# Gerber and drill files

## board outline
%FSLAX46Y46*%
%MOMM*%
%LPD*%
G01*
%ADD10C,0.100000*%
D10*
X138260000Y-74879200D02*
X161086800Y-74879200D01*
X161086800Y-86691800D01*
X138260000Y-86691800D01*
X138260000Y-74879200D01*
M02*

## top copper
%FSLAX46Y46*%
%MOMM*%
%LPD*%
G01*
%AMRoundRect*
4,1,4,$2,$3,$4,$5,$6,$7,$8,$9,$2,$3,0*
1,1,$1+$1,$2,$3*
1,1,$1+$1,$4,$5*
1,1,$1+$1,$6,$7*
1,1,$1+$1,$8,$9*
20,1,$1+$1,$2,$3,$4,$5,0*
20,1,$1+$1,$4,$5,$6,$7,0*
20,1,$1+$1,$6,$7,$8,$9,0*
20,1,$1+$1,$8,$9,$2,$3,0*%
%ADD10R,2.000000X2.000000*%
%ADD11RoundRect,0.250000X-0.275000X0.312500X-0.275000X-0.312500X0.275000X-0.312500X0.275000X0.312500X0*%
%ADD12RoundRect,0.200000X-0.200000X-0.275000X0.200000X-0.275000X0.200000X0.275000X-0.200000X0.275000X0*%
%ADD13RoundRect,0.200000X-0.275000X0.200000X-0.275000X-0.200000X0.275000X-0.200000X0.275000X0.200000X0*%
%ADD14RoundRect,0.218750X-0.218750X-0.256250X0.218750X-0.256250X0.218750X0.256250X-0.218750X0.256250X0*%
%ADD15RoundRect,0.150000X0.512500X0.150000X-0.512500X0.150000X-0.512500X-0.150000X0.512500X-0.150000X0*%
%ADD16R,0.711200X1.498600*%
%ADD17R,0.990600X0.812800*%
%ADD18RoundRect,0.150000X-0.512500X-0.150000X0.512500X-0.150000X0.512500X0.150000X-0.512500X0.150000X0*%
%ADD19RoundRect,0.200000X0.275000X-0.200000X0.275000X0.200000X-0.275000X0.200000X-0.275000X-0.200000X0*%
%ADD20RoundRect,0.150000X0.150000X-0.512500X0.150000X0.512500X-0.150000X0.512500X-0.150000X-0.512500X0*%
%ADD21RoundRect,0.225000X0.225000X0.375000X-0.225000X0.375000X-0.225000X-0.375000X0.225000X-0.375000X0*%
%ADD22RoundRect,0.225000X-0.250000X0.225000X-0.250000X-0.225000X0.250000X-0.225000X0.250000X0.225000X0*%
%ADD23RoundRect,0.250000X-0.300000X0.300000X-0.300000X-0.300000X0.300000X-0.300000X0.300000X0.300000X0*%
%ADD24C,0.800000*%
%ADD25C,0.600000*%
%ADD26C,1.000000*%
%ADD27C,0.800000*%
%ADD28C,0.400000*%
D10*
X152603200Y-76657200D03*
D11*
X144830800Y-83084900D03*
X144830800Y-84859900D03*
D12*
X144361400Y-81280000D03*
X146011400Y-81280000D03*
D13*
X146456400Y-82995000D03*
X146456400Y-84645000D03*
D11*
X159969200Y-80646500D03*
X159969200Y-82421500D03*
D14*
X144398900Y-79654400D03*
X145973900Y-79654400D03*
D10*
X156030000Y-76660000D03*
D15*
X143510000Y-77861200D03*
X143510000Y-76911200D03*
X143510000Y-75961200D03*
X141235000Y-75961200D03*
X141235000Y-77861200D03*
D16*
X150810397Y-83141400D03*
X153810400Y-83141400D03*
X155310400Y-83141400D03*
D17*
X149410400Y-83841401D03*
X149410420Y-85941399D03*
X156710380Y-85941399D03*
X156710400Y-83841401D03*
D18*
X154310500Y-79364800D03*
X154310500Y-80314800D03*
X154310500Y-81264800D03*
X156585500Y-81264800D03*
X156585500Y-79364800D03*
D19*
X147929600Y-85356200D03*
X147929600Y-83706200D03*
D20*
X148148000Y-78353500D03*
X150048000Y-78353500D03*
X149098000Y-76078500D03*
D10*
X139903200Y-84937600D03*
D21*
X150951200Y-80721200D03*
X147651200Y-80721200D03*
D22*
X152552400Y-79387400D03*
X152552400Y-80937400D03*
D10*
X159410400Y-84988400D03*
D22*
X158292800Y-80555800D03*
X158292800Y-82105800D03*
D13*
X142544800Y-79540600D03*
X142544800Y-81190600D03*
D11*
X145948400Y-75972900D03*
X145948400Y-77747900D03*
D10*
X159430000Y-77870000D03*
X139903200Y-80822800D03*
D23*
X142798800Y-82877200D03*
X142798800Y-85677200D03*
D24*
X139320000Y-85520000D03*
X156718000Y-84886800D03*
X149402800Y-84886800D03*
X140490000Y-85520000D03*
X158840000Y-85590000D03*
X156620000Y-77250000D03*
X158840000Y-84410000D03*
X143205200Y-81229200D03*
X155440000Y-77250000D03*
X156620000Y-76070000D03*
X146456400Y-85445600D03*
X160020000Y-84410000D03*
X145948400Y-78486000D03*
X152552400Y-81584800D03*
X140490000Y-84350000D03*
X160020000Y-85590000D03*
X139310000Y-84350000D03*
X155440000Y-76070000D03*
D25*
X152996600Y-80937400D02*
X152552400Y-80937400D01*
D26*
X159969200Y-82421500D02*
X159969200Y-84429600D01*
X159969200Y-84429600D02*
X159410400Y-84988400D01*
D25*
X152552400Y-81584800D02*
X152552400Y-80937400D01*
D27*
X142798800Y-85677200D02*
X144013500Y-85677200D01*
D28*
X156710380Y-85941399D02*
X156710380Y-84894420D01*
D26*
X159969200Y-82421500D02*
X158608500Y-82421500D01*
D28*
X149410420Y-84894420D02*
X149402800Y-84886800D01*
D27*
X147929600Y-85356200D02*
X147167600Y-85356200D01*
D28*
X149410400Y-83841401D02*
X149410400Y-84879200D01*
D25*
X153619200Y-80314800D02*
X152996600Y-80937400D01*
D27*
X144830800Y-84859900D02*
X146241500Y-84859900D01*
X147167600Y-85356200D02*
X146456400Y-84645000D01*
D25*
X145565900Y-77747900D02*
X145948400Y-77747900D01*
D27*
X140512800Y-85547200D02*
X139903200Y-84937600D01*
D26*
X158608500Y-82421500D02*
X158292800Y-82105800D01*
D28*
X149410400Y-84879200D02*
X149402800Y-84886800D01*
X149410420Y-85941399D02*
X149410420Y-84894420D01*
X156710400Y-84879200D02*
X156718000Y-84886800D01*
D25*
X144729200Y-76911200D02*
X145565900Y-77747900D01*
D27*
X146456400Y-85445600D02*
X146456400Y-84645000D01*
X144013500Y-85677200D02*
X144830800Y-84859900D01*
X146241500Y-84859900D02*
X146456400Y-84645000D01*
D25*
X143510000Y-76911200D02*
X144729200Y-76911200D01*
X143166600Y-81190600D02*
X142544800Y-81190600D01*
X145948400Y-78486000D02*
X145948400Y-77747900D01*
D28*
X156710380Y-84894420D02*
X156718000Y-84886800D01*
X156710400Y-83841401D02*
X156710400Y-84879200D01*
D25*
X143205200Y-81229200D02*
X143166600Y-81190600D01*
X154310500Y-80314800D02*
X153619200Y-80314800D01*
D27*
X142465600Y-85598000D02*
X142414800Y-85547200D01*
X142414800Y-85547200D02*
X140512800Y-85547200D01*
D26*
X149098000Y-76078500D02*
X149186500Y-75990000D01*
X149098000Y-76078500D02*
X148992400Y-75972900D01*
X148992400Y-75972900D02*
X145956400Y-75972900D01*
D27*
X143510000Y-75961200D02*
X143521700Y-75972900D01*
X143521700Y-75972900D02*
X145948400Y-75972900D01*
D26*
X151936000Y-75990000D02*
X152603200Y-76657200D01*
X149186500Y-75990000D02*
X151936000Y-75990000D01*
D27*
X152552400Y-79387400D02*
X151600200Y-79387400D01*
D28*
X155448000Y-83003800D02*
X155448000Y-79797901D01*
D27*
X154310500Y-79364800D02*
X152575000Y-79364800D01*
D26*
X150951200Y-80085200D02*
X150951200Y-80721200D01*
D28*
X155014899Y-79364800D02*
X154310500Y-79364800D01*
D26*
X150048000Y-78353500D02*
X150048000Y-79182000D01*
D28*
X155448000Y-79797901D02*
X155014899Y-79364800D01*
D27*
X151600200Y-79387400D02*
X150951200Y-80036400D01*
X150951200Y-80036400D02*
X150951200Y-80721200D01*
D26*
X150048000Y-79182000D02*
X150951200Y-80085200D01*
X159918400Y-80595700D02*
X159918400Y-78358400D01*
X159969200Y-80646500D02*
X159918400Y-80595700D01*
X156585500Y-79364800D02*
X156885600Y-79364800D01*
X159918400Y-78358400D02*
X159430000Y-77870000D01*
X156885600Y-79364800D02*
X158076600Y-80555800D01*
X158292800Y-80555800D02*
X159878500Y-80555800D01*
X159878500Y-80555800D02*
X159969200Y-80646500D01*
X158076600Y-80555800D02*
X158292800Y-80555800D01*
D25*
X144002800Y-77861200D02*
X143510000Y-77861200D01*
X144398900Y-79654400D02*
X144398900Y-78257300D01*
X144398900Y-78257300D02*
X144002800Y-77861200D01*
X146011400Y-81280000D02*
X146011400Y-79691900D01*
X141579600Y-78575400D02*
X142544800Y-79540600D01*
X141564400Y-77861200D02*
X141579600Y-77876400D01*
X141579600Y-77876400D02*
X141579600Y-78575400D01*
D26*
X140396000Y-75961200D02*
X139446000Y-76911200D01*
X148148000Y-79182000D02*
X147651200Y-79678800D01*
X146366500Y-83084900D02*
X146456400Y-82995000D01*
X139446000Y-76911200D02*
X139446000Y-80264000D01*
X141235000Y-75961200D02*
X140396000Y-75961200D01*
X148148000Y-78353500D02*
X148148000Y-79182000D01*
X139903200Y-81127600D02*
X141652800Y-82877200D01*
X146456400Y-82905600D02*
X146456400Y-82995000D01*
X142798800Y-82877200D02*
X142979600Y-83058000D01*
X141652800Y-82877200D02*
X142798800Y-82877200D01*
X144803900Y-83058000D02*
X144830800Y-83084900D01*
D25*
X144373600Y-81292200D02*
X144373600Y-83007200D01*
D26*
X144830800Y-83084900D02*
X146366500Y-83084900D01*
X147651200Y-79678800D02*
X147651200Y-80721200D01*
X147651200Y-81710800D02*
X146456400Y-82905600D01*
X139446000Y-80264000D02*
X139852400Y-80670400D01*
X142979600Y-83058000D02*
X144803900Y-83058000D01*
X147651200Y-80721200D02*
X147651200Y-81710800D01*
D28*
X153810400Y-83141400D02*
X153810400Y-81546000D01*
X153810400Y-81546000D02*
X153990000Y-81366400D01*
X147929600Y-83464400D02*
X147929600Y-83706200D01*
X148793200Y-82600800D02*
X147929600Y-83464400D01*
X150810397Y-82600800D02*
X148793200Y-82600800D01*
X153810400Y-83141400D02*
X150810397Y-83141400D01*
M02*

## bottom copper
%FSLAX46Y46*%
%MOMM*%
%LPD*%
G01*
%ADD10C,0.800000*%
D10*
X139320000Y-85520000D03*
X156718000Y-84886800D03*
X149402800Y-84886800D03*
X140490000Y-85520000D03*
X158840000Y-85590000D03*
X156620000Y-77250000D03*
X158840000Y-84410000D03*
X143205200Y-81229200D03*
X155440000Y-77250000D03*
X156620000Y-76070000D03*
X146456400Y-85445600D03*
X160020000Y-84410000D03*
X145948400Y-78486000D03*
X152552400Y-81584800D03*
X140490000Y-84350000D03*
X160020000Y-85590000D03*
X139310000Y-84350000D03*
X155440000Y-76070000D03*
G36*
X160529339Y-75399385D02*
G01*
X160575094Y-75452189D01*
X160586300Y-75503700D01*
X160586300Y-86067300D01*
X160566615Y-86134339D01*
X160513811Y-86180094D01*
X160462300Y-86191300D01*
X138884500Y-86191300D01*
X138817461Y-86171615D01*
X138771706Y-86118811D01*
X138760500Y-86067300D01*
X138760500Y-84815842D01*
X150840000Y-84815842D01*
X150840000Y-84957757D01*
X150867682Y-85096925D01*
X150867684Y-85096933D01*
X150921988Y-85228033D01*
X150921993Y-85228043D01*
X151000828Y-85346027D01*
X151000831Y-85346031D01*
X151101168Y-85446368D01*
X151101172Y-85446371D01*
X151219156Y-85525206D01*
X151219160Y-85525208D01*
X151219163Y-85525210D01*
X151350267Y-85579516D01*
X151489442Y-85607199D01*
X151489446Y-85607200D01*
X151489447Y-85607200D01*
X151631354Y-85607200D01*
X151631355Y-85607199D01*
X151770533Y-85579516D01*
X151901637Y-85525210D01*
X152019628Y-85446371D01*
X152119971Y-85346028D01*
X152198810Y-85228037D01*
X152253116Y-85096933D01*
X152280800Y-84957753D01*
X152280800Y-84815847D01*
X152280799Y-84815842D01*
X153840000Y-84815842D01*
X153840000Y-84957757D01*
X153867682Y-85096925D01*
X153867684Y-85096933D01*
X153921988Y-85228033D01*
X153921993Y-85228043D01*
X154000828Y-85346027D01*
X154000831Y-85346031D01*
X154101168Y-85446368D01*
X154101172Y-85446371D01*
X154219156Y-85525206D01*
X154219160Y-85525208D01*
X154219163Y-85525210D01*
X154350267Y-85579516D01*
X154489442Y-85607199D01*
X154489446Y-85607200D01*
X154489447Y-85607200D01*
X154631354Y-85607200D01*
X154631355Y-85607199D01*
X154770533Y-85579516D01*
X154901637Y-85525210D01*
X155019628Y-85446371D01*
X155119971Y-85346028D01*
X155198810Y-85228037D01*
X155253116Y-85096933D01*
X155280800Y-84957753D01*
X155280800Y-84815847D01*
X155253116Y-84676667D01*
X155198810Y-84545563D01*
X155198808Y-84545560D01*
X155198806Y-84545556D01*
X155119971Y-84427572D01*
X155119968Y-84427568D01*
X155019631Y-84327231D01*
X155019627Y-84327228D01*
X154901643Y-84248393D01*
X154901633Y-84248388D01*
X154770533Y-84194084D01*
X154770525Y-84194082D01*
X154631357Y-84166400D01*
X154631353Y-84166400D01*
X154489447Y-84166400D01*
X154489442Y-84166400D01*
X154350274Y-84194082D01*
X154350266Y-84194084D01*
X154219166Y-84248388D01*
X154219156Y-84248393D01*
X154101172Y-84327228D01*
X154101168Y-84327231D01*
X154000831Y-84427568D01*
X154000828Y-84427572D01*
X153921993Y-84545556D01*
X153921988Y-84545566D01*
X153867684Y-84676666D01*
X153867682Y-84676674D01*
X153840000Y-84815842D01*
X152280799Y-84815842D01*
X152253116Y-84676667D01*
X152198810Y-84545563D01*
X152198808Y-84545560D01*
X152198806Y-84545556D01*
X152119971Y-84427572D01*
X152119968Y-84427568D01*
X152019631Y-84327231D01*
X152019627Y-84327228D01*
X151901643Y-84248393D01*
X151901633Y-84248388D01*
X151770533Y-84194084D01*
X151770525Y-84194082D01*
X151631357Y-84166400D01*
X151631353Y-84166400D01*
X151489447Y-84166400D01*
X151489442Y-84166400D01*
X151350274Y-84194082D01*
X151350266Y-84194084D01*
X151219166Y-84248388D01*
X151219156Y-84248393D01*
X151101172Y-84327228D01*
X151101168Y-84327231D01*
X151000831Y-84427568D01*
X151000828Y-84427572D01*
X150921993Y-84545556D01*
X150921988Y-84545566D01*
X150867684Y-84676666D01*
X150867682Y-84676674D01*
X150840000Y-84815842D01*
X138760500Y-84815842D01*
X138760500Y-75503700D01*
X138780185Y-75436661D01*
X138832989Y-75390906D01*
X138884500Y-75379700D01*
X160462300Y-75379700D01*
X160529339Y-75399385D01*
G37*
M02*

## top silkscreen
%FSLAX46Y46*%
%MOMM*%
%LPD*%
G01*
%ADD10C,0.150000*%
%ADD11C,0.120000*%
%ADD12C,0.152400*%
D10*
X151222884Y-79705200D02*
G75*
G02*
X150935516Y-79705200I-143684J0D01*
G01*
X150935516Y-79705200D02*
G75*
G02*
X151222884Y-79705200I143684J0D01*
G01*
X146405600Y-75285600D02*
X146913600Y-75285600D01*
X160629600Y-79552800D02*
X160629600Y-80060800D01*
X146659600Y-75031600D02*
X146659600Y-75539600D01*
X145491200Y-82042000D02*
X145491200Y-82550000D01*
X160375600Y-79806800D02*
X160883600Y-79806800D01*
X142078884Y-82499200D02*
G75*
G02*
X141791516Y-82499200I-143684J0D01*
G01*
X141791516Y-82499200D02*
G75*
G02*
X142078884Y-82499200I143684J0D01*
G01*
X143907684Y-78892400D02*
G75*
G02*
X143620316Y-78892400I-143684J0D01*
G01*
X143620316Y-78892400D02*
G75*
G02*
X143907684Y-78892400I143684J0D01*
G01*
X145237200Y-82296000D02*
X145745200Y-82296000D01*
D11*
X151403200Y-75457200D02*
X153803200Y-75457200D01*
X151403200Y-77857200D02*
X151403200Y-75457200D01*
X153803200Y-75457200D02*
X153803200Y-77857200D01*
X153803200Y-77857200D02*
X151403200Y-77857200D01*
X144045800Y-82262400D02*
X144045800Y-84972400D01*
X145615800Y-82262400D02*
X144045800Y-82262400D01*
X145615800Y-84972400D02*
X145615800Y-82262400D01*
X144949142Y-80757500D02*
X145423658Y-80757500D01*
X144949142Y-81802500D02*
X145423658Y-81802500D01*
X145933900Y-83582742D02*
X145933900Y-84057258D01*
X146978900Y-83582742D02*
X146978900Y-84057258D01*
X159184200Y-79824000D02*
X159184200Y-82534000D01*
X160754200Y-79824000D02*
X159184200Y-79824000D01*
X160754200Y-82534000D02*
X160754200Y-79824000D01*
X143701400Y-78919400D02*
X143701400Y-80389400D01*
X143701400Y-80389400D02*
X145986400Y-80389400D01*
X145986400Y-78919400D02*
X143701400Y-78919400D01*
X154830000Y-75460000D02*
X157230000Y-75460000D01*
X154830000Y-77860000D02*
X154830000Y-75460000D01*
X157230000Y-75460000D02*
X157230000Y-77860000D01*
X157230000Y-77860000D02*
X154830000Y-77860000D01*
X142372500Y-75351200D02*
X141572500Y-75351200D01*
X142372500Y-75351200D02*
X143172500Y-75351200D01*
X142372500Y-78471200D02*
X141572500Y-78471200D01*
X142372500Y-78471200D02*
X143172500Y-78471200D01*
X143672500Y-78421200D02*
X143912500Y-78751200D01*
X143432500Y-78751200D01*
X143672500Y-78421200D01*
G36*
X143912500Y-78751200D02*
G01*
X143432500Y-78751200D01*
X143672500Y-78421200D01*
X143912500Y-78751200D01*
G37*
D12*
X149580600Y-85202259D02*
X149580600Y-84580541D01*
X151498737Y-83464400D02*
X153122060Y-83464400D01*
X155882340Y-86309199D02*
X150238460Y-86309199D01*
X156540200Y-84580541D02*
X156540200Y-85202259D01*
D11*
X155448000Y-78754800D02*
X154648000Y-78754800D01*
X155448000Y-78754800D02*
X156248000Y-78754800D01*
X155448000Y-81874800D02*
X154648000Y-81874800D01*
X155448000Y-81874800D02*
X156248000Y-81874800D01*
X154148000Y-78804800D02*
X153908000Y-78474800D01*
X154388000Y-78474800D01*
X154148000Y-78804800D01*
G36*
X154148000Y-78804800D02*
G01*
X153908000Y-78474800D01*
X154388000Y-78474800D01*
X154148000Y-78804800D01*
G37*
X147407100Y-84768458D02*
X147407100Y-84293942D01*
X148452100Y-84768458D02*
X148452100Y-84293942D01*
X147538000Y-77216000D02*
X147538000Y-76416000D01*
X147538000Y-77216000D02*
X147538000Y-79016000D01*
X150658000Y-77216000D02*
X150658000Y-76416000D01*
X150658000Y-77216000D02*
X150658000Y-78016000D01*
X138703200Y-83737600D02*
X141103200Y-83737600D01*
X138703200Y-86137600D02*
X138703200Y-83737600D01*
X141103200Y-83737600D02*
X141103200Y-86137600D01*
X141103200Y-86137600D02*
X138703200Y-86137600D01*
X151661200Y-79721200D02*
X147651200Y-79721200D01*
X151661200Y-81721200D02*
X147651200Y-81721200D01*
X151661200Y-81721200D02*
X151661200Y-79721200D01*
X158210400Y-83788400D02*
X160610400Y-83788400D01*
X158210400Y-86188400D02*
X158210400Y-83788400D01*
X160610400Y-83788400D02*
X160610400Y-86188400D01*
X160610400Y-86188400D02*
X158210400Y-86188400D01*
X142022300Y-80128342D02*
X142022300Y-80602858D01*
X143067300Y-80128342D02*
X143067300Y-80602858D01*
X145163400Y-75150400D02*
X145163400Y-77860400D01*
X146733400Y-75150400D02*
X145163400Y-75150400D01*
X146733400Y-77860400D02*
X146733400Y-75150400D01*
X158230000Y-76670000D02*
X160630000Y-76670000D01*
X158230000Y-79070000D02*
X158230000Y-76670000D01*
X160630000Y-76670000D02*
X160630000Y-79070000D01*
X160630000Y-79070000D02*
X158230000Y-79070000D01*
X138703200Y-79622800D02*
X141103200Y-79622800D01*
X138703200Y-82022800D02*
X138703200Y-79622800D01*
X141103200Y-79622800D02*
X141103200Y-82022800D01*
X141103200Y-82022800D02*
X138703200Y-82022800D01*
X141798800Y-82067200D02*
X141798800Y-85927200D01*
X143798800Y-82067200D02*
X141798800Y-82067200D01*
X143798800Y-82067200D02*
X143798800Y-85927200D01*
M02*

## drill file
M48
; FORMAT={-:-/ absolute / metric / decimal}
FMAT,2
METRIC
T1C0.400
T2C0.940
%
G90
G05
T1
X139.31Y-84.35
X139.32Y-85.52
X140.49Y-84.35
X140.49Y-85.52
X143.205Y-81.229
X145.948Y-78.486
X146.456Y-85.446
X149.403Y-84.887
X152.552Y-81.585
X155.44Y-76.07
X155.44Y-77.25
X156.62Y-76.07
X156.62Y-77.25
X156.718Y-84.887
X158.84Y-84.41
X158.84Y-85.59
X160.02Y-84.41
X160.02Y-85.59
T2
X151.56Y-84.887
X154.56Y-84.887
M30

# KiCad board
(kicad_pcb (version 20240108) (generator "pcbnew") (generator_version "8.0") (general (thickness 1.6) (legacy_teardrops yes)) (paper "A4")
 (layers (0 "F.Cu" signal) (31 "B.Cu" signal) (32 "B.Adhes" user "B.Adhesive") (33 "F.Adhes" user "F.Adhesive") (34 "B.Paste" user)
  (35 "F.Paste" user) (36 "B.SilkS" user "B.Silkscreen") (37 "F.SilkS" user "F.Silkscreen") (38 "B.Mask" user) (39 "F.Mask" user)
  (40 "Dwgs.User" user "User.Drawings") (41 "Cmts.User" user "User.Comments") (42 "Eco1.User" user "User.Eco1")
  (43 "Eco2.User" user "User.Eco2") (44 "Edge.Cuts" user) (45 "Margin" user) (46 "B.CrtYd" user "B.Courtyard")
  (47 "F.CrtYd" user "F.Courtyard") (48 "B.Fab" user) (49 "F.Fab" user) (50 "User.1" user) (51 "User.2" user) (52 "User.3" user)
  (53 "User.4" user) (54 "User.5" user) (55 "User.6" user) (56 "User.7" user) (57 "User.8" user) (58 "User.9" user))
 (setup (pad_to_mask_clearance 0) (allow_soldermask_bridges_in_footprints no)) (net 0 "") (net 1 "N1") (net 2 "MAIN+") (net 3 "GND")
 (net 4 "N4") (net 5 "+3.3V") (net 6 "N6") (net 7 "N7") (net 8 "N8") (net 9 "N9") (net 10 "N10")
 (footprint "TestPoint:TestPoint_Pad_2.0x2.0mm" (layer "F.Cu") (at 152.6032 76.6572)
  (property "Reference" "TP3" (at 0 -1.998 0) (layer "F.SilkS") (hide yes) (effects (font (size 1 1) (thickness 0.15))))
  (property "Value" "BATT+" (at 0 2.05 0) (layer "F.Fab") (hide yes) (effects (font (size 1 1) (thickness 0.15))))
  (fp_line (start -1.2 -1.2) (end 1.2 -1.2) (stroke (width 0.12) (type solid)) (layer "F.SilkS"))
  (fp_line (start -1.2 1.2) (end -1.2 -1.2) (stroke (width 0.12) (type solid)) (layer "F.SilkS"))
  (fp_line (start 1.2 -1.2) (end 1.2 1.2) (stroke (width 0.12) (type solid)) (layer "F.SilkS"))
  (fp_line (start 1.2 1.2) (end -1.2 1.2) (stroke (width 0.12) (type solid)) (layer "F.SilkS"))
  (pad "1" smd rect (at 0 0) (size 2 2) (layers "F.Cu" "F.Mask") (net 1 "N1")))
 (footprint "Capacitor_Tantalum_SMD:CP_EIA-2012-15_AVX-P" (layer "F.Cu") (at 144.8308 83.9724 -90)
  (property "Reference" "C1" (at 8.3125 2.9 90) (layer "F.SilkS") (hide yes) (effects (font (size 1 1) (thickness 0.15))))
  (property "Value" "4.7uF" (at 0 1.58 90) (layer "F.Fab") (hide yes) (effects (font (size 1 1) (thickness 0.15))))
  (fp_line (start -1.71 0.785) (end 1 0.785) (stroke (width 0.12) (type solid)) (layer "F.SilkS"))
  (fp_line (start -1.71 -0.785) (end -1.71 0.785) (stroke (width 0.12) (type solid)) (layer "F.SilkS"))
  (fp_line (start 1 -0.785) (end -1.71 -0.785) (stroke (width 0.12) (type solid)) (layer "F.SilkS"))
  (pad "1" smd roundrect (at -0.8875 0 270) (size 1.125 1.05) (layers "F.Cu" "F.Paste" "F.Mask") (roundrect_rratio 0.238095) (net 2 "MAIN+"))
  (pad "2" smd roundrect (at 0.8875 0 270) (size 1.125 1.05) (layers "F.Cu" "F.Paste" "F.Mask") (roundrect_rratio 0.238095) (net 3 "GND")))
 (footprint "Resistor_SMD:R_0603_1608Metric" (layer "F.Cu") (at 145.1864 81.28)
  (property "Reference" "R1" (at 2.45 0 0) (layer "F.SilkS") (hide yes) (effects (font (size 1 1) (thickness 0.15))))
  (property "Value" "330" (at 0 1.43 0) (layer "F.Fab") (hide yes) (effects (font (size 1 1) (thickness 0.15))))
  (fp_line (start -0.237258 -0.5225) (end 0.237258 -0.5225) (stroke (width 0.12) (type solid)) (layer "F.SilkS"))
  (fp_line (start -0.237258 0.5225) (end 0.237258 0.5225) (stroke (width 0.12) (type solid)) (layer "F.SilkS"))
  (pad "1" smd roundrect (at -0.825 0) (size 0.8 0.95) (layers "F.Cu" "F.Paste" "F.Mask") (roundrect_rratio 0.25) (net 2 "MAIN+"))
  (pad "2" smd roundrect (at 0.825 0) (size 0.8 0.95) (layers "F.Cu" "F.Paste" "F.Mask") (roundrect_rratio 0.25) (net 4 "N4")))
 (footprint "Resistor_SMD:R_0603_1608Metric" (layer "F.Cu") (at 146.4564 83.82 -90)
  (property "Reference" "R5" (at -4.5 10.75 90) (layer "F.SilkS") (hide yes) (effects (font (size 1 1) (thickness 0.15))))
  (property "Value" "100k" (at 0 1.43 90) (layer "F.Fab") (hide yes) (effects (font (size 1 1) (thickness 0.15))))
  (fp_line (start -0.237258 0.5225) (end 0.237258 0.5225) (stroke (width 0.12) (type solid)) (layer "F.SilkS"))
  (fp_line (start -0.237258 -0.5225) (end 0.237258 -0.5225) (stroke (width 0.12) (type solid)) (layer "F.SilkS"))
  (pad "1" smd roundrect (at -0.825 0 270) (size 0.8 0.95) (layers "F.Cu" "F.Paste" "F.Mask") (roundrect_rratio 0.25) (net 2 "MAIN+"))
  (pad "2" smd roundrect (at 0.825 0 270) (size 0.8 0.95) (layers "F.Cu" "F.Paste" "F.Mask") (roundrect_rratio 0.25) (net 3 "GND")))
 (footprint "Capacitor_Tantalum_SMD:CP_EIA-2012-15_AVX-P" (layer "F.Cu") (at 159.9692 81.534 -90)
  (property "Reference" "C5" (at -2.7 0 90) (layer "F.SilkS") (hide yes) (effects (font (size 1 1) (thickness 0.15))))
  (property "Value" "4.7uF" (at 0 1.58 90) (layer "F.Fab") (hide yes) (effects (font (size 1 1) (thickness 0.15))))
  (fp_line (start -1.71 0.785) (end 1 0.785) (stroke (width 0.12) (type solid)) (layer "F.SilkS"))
  (fp_line (start -1.71 -0.785) (end -1.71 0.785) (stroke (width 0.12) (type solid)) (layer "F.SilkS"))
  (fp_line (start 1 -0.785) (end -1.71 -0.785) (stroke (width 0.12) (type solid)) (layer "F.SilkS"))
  (pad "1" smd roundrect (at -0.8875 0 270) (size 1.125 1.05) (layers "F.Cu" "F.Paste" "F.Mask") (roundrect_rratio 0.238095) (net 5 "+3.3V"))
  (pad "2" smd roundrect (at 0.8875 0 270) (size 1.125 1.05) (layers "F.Cu" "F.Paste" "F.Mask") (roundrect_rratio 0.238095) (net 3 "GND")))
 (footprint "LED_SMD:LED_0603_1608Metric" (layer "F.Cu") (at 145.1864 79.6544)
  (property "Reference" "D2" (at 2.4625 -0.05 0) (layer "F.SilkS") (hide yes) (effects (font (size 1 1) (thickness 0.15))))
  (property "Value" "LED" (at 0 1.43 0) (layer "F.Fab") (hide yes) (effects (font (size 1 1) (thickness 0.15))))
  (fp_line (start -1.485 -0.735) (end -1.485 0.735) (stroke (width 0.12) (type solid)) (layer "F.SilkS"))
  (fp_line (start -1.485 0.735) (end 0.8 0.735) (stroke (width 0.12) (type solid)) (layer "F.SilkS"))
  (fp_line (start 0.8 -0.735) (end -1.485 -0.735) (stroke (width 0.12) (type solid)) (layer "F.SilkS"))
  (pad "1" smd roundrect (at -0.7875 0) (size 0.875 0.95) (layers "F.Cu" "F.Paste" "F.Mask") (roundrect_rratio 0.25) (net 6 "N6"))
  (pad "2" smd roundrect (at 0.7875 0) (size 0.875 0.95) (layers "F.Cu" "F.Paste" "F.Mask") (roundrect_rratio 0.25) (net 4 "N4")))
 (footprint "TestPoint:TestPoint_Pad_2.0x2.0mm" (layer "F.Cu") (at 156.03 76.66)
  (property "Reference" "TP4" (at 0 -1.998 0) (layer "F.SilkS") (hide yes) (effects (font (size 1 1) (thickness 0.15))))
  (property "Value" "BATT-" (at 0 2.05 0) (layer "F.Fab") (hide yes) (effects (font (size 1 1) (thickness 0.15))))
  (fp_line (start -1.2 -1.2) (end 1.2 -1.2) (stroke (width 0.12) (type solid)) (layer "F.SilkS"))
  (fp_line (start -1.2 1.2) (end -1.2 -1.2) (stroke (width 0.12) (type solid)) (layer "F.SilkS"))
  (fp_line (start 1.2 -1.2) (end 1.2 1.2) (stroke (width 0.12) (type solid)) (layer "F.SilkS"))
  (fp_line (start 1.2 1.2) (end -1.2 1.2) (stroke (width 0.12) (type solid)) (layer "F.SilkS"))
  (pad "1" smd rect (at 0 0) (size 2 2) (layers "F.Cu" "F.Mask") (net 3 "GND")))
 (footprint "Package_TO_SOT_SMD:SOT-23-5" (layer "F.Cu") (at 142.3725 76.9112 180)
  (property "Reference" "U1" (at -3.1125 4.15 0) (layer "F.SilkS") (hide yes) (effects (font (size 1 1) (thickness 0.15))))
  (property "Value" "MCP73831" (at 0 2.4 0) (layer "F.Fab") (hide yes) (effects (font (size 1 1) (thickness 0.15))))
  (fp_line (start 0 1.56) (end 0.8 1.56) (stroke (width 0.12) (type solid)) (layer "F.SilkS"))
  (fp_line (start 0 1.56) (end -0.8 1.56) (stroke (width 0.12) (type solid)) (layer "F.SilkS"))
  (fp_line (start 0 -1.56) (end 0.8 -1.56) (stroke (width 0.12) (type solid)) (layer "F.SilkS"))
  (fp_line (start 0 -1.56) (end -0.8 -1.56) (stroke (width 0.12) (type solid)) (layer "F.SilkS"))
  (fp_poly
   (pts (xy -1.3 -1.51) (xy -1.54 -1.84) (xy -1.06 -1.84) (xy -1.3 -1.51)) (stroke (width 0.12) (type solid)) (fill solid) (layer "F.SilkS"))
  (pad "1" smd roundrect (at -1.1375 -0.95 180) (size 1.325 0.6) (layers "F.Cu" "F.Paste" "F.Mask") (roundrect_rratio 0.25) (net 6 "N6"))
  (pad "2" smd roundrect (at -1.1375 0 180) (size 1.325 0.6) (layers "F.Cu" "F.Paste" "F.Mask") (roundrect_rratio 0.25) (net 3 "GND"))
  (pad "3" smd roundrect (at -1.1375 0.95 180) (size 1.325 0.6) (layers "F.Cu" "F.Paste" "F.Mask") (roundrect_rratio 0.25) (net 1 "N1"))
  (pad "4" smd roundrect (at 1.1375 0.95 180) (size 1.325 0.6) (layers "F.Cu" "F.Paste" "F.Mask") (roundrect_rratio 0.25) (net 2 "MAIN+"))
  (pad "5" smd roundrect (at 1.1375 -0.95 180) (size 1.325 0.6) (layers "F.Cu" "F.Paste" "F.Mask") (roundrect_rratio 0.25) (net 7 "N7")))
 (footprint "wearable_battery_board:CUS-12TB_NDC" (layer "F.Cu") (at 153.0604 84.8868)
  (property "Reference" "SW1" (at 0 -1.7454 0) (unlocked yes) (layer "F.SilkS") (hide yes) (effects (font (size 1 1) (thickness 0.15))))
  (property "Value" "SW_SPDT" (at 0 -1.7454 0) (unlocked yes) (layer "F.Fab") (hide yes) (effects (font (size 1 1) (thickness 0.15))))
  (fp_line (start -3.4798 0.315459) (end -3.4798 -0.306259) (stroke (width 0.1524) (type solid)) (layer "F.SilkS"))
  (fp_line (start -1.561663 -1.4224) (end 0.06166 -1.4224) (stroke (width 0.1524) (type solid)) (layer "F.SilkS"))
  (fp_line (start 2.82194 1.422399) (end -2.82194 1.422399) (stroke (width 0.1524) (type solid)) (layer "F.SilkS"))
  (fp_line (start 3.4798 -0.306259) (end 3.4798 0.315459) (stroke (width 0.1524) (type solid)) (layer "F.SilkS"))
  (pad "" np_thru_hole circle (at -1.5 0) (size 0.9398 0.9398) (drill 0.9398) (layers))
  (pad "" np_thru_hole circle (at 1.5 0) (size 0.9398 0.9398) (drill 0.9398) (layers))
  (pad "1" smd rect (at -2.250003 -1.7454) (size 0.7112 1.4986) (layers "F.Cu" "F.Paste" "F.Mask") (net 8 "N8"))
  (pad "2" smd rect (at 0.75 -1.7454) (size 0.7112 1.4986) (layers "F.Cu" "F.Paste" "F.Mask") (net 8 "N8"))
  (pad "3" smd rect (at 2.25 -1.7454) (size 0.7112 1.4986) (layers "F.Cu" "F.Paste" "F.Mask") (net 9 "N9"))
  (pad "4" smd rect (at -3.65 -1.045399) (size 0.9906 0.8128) (layers "F.Cu" "F.Paste" "F.Mask") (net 3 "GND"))
  (pad "4" smd rect (at -3.64998 1.054599) (size 0.9906 0.8128) (layers "F.Cu" "F.Paste" "F.Mask") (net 3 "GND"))
  (pad "4" smd rect (at 3.64998 1.054599) (size 0.9906 0.8128) (layers "F.Cu" "F.Paste" "F.Mask") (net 3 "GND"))
  (pad "4" smd rect (at 3.65 -1.045399) (size 0.9906 0.8128) (layers "F.Cu" "F.Paste" "F.Mask") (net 3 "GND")))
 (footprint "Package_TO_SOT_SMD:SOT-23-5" (layer "F.Cu") (at 155.448 80.3148)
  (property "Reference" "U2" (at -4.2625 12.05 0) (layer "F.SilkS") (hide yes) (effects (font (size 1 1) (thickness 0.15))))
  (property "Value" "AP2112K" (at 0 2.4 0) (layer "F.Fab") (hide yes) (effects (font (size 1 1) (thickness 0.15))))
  (fp_line (start 0 -1.56) (end -0.8 -1.56) (stroke (width 0.12) (type solid)) (layer "F.SilkS"))
  (fp_line (start 0 -1.56) (end 0.8 -1.56) (stroke (width 0.12) (type solid)) (layer "F.SilkS"))
  (fp_line (start 0 1.56) (end -0.8 1.56) (stroke (width 0.12) (type solid)) (layer "F.SilkS"))
  (fp_line (start 0 1.56) (end 0.8 1.56) (stroke (width 0.12) (type solid)) (layer "F.SilkS"))
  (fp_poly
   (pts (xy -1.3 -1.51) (xy -1.54 -1.84) (xy -1.06 -1.84) (xy -1.3 -1.51)) (stroke (width 0.12) (type solid)) (fill solid) (layer "F.SilkS"))
  (pad "1" smd roundrect (at -1.1375 -0.95) (size 1.325 0.6) (layers "F.Cu" "F.Paste" "F.Mask") (roundrect_rratio 0.25) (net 9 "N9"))
  (pad "2" smd roundrect (at -1.1375 0) (size 1.325 0.6) (layers "F.Cu" "F.Paste" "F.Mask") (roundrect_rratio 0.25) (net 3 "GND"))
  (pad "3" smd roundrect (at -1.1375 0.95) (size 1.325 0.6) (layers "F.Cu" "F.Paste" "F.Mask") (roundrect_rratio 0.25) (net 8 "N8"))
  (pad "4" smd roundrect (at 1.1375 0.95) (size 1.325 0.6) (layers "F.Cu" "F.Paste" "F.Mask") (roundrect_rratio 0.25) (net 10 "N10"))
  (pad "5" smd roundrect (at 1.1375 -0.95) (size 1.325 0.6) (layers "F.Cu" "F.Paste" "F.Mask") (roundrect_rratio 0.25) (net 5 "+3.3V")))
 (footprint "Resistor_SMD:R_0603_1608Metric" (layer "F.Cu") (at 147.9296 84.5312 90)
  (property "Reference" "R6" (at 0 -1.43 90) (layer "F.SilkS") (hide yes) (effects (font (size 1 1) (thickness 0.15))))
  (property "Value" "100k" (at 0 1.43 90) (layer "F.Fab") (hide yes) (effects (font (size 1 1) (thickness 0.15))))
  (fp_line (start -0.237258 -0.5225) (end 0.237258 -0.5225) (stroke (width 0.12) (type solid)) (layer "F.SilkS"))
  (fp_line (start -0.237258 0.5225) (end 0.237258 0.5225) (stroke (width 0.12) (type solid)) (layer "F.SilkS"))
  (pad "1" smd roundrect (at -0.825 0 90) (size 0.8 0.95) (layers "F.Cu" "F.Paste" "F.Mask") (roundrect_rratio 0.25) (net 3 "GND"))
  (pad "2" smd roundrect (at 0.825 0 90) (size 0.8 0.95) (layers "F.Cu" "F.Paste" "F.Mask") (roundrect_rratio 0.25) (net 8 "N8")))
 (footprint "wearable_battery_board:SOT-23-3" (layer "F.Cu") (at 149.098 77.216 90)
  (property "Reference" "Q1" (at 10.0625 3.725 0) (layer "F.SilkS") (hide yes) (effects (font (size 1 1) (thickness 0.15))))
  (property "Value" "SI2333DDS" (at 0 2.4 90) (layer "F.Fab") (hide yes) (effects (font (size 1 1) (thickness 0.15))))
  (fp_line (start 0 -1.56) (end 0.8 -1.56) (stroke (width 0.12) (type solid)) (layer "F.SilkS"))
  (fp_line (start 0 -1.56) (end -1.8 -1.56) (stroke (width 0.12) (type solid)) (layer "F.SilkS"))
  (fp_line (start 0 1.56) (end 0.8 1.56) (stroke (width 0.12) (type solid)) (layer "F.SilkS"))
  (fp_line (start 0 1.56) (end -0.8 1.56) (stroke (width 0.12) (type solid)) (layer "F.SilkS"))
  (pad "1" smd roundrect (at -1.1375 -0.95 90) (size 1.325 0.6) (layers "F.Cu" "F.Paste" "F.Mask") (roundrect_rratio 0.25) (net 2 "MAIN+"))
  (pad "2" smd roundrect (at -1.1375 0.95 90) (size 1.325 0.6) (layers "F.Cu" "F.Paste" "F.Mask") (roundrect_rratio 0.25) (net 9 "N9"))
  (pad "3" smd roundrect (at 1.1375 0 90) (size 1.325 0.6) (layers "F.Cu" "F.Paste" "F.Mask") (roundrect_rratio 0.25) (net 1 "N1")))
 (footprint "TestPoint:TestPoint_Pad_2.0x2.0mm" (layer "F.Cu") (at 139.9032 84.9376 90)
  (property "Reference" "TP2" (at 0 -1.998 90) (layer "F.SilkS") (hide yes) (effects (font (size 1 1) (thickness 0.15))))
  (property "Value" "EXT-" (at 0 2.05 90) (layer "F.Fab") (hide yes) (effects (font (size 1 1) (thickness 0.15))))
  (fp_line (start 1.2 -1.2) (end 1.2 1.2) (stroke (width 0.12) (type solid)) (layer "F.SilkS"))
  (fp_line (start -1.2 -1.2) (end 1.2 -1.2) (stroke (width 0.12) (type solid)) (layer "F.SilkS"))
  (fp_line (start 1.2 1.2) (end -1.2 1.2) (stroke (width 0.12) (type solid)) (layer "F.SilkS"))
  (fp_line (start -1.2 1.2) (end -1.2 -1.2) (stroke (width 0.12) (type solid)) (layer "F.SilkS"))
  (pad "1" smd rect (at 0 0 90) (size 2 2) (layers "F.Cu" "F.Mask") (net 3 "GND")))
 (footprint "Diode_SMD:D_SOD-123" (layer "F.Cu") (at 149.3012 80.7212 180)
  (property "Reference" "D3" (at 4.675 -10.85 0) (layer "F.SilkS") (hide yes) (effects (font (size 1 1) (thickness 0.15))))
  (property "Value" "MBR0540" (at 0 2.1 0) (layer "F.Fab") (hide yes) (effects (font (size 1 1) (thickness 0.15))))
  (fp_line (start -2.36 1) (end 1.65 1) (stroke (width 0.12) (type solid)) (layer "F.SilkS"))
  (fp_line (start -2.36 -1) (end 1.65 -1) (stroke (width 0.12) (type solid)) (layer "F.SilkS"))
  (fp_line (start -2.36 -1) (end -2.36 1) (stroke (width 0.12) (type solid)) (layer "F.SilkS"))
  (pad "1" smd roundrect (at -1.65 0 180) (size 0.9 1.2) (layers "F.Cu" "F.Paste" "F.Mask") (roundrect_rratio 0.25) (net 9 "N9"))
  (pad "2" smd roundrect (at 1.65 0 180) (size 0.9 1.2) (layers "F.Cu" "F.Paste" "F.Mask") (roundrect_rratio 0.25) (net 2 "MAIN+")))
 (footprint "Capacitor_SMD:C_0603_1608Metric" (layer "F.Cu") (at 152.5524 80.1624 -90)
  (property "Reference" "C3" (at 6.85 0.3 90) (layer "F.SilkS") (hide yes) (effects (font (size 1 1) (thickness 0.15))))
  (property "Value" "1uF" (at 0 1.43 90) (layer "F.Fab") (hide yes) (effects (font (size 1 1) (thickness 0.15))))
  (pad "1" smd roundrect (at -0.775 0 270) (size 0.9 0.95) (layers "F.Cu" "F.Paste" "F.Mask") (roundrect_rratio 0.25) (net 9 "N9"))
  (pad "2" smd roundrect (at 0.775 0 270) (size 0.9 0.95) (layers "F.Cu" "F.Paste" "F.Mask") (roundrect_rratio 0.25) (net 3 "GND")))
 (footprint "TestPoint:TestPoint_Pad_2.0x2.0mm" (layer "F.Cu") (at 159.4104 84.9884)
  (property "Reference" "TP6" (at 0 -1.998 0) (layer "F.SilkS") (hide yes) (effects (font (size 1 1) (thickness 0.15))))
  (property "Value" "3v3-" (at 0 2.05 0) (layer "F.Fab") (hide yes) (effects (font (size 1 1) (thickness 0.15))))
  (fp_line (start -1.2 -1.2) (end 1.2 -1.2) (stroke (width 0.12) (type solid)) (layer "F.SilkS"))
  (fp_line (start -1.2 1.2) (end -1.2 -1.2) (stroke (width 0.12) (type solid)) (layer "F.SilkS"))
  (fp_line (start 1.2 -1.2) (end 1.2 1.2) (stroke (width 0.12) (type solid)) (layer "F.SilkS"))
  (fp_line (start 1.2 1.2) (end -1.2 1.2) (stroke (width 0.12) (type solid)) (layer "F.SilkS"))
  (pad "1" smd rect (at 0 0) (size 2 2) (layers "F.Cu" "F.Mask") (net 3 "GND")))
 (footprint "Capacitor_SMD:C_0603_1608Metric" (layer "F.Cu") (at 158.2928 81.3308 -90)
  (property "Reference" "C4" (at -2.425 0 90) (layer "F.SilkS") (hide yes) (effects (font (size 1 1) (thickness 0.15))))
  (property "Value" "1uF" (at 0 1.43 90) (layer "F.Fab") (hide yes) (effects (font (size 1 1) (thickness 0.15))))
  (pad "1" smd roundrect (at -0.775 0 270) (size 0.9 0.95) (layers "F.Cu" "F.Paste" "F.Mask") (roundrect_rratio 0.25) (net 5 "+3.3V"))
  (pad "2" smd roundrect (at 0.775 0 270) (size 0.9 0.95) (layers "F.Cu" "F.Paste" "F.Mask") (roundrect_rratio 0.25) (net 3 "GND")))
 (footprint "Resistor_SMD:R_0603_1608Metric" (layer "F.Cu") (at 142.5448 80.3656 -90)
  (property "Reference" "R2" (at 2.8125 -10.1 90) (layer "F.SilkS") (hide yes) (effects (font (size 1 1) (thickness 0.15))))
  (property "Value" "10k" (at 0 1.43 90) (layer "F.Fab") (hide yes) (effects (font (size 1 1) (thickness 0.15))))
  (fp_line (start -0.237258 0.5225) (end 0.237258 0.5225) (stroke (width 0.12) (type solid)) (layer "F.SilkS"))
  (fp_line (start -0.237258 -0.5225) (end 0.237258 -0.5225) (stroke (width 0.12) (type solid)) (layer "F.SilkS"))
  (pad "1" smd roundrect (at -0.825 0 270) (size 0.8 0.95) (layers "F.Cu" "F.Paste" "F.Mask") (roundrect_rratio 0.25) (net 7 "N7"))
  (pad "2" smd roundrect (at 0.825 0 270) (size 0.8 0.95) (layers "F.Cu" "F.Paste" "F.Mask") (roundrect_rratio 0.25) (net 3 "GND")))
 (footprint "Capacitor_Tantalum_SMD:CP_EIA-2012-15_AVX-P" (layer "F.Cu") (at 145.9484 76.8604 -90)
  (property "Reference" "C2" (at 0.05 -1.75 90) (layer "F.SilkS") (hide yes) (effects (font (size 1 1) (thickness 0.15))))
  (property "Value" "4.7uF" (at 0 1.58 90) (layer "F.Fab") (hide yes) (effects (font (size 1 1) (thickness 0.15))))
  (fp_line (start -1.71 0.785) (end 1 0.785) (stroke (width 0.12) (type solid)) (layer "F.SilkS"))
  (fp_line (start -1.71 -0.785) (end -1.71 0.785) (stroke (width 0.12) (type solid)) (layer "F.SilkS"))
  (fp_line (start 1 -0.785) (end -1.71 -0.785) (stroke (width 0.12) (type solid)) (layer "F.SilkS"))
  (pad "1" smd roundrect (at -0.8875 0 270) (size 1.125 1.05) (layers "F.Cu" "F.Paste" "F.Mask") (roundrect_rratio 0.238095) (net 1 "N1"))
  (pad "2" smd roundrect (at 0.8875 0 270) (size 1.125 1.05) (layers "F.Cu" "F.Paste" "F.Mask") (roundrect_rratio 0.238095) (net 3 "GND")))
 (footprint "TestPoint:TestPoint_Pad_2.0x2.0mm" (layer "F.Cu") (at 159.43 77.87)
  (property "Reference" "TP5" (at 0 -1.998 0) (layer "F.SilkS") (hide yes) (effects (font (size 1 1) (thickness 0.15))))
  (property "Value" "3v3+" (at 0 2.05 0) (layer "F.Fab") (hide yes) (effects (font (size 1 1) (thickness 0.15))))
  (fp_line (start -1.2 -1.2) (end 1.2 -1.2) (stroke (width 0.12) (type solid)) (layer "F.SilkS"))
  (fp_line (start -1.2 1.2) (end -1.2 -1.2) (stroke (width 0.12) (type solid)) (layer "F.SilkS"))
  (fp_line (start 1.2 -1.2) (end 1.2 1.2) (stroke (width 0.12) (type solid)) (layer "F.SilkS"))
  (fp_line (start 1.2 1.2) (end -1.2 1.2) (stroke (width 0.12) (type solid)) (layer "F.SilkS"))
  (pad "1" smd rect (at 0 0) (size 2 2) (layers "F.Cu" "F.Mask") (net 5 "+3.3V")))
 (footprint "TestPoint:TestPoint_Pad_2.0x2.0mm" (layer "F.Cu") (at 139.9032 80.8228)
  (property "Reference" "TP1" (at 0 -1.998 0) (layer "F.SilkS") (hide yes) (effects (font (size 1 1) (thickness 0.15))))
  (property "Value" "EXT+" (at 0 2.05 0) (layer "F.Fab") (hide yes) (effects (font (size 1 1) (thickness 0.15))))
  (fp_line (start -1.2 -1.2) (end 1.2 -1.2) (stroke (width 0.12) (type solid)) (layer "F.SilkS"))
  (fp_line (start -1.2 1.2) (end -1.2 -1.2) (stroke (width 0.12) (type solid)) (layer "F.SilkS"))
  (fp_line (start 1.2 -1.2) (end 1.2 1.2) (stroke (width 0.12) (type solid)) (layer "F.SilkS"))
  (fp_line (start 1.2 1.2) (end -1.2 1.2) (stroke (width 0.12) (type solid)) (layer "F.SilkS"))
  (pad "1" smd rect (at 0 0) (size 2 2) (layers "F.Cu" "F.Mask") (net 2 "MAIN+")))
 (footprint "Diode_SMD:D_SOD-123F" (layer "F.Cu") (at 142.7988 84.2772 -90)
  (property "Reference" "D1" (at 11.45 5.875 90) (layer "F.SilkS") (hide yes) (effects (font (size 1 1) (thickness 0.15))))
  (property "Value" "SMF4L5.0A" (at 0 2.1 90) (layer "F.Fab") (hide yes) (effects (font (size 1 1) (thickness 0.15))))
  (fp_line (start -2.21 1) (end 1.65 1) (stroke (width 0.12) (type solid)) (layer "F.SilkS"))
  (fp_line (start -2.21 -1) (end -2.21 1) (stroke (width 0.12) (type solid)) (layer "F.SilkS"))
  (fp_line (start -2.21 -1) (end 1.65 -1) (stroke (width 0.12) (type solid)) (layer "F.SilkS"))
  (pad "1" smd roundrect (at -1.4 0 270) (size 1.1 1.1) (layers "F.Cu" "F.Paste" "F.Mask") (roundrect_rratio 0.2272727273) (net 2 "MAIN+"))
  (pad "2" smd roundrect (at 1.4 0 270) (size 1.1 1.1) (layers "F.Cu" "F.Paste" "F.Mask") (roundrect_rratio 0.2272727273) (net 3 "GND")))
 (gr_circle (center 151.0792 79.7052) (end 151.1808 79.8068) (stroke (width 0.15) (type default)) (fill none) (layer "F.SilkS"))
 (gr_line (start 146.4056 75.2856) (end 146.9136 75.2856) (stroke (width 0.15) (type default)) (layer "F.SilkS"))
 (gr_line (start 160.6296 79.5528) (end 160.6296 80.0608) (stroke (width 0.15) (type default)) (layer "F.SilkS"))
 (gr_line (start 146.6596 75.0316) (end 146.6596 75.5396) (stroke (width 0.15) (type default)) (layer "F.SilkS"))
 (gr_line (start 145.4912 82.042) (end 145.4912 82.55) (stroke (width 0.15) (type default)) (layer "F.SilkS"))
 (gr_line (start 160.3756 79.8068) (end 160.8836 79.8068) (stroke (width 0.15) (type default)) (layer "F.SilkS"))
 (gr_circle (center 141.9352 82.4992) (end 142.0368 82.6008) (stroke (width 0.15) (type default)) (fill none) (layer "F.SilkS"))
 (gr_circle (center 143.764 78.8924) (end 143.8656 78.994) (stroke (width 0.15) (type default)) (fill none) (layer "F.SilkS"))
 (gr_line (start 145.2372 82.296) (end 145.7452 82.296) (stroke (width 0.15) (type default)) (layer "F.SilkS"))
 (gr_rect (start 138.26 74.8792) (end 161.0868 86.6918) (stroke (width 0.1) (type default)) (fill none) (layer "Edge.Cuts"))
 (segment (start 152.9966 80.9374) (end 152.5524 80.9374) (width 0.6) (layer "F.Cu") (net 3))
 (segment (start 159.9692 82.4215) (end 159.9692 84.4296) (width 1) (layer "F.Cu") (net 3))
 (segment (start 159.9692 84.4296) (end 159.4104 84.9884) (width 1) (layer "F.Cu") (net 3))
 (segment (start 152.5524 81.5848) (end 152.5524 80.9374) (width 0.6) (layer "F.Cu") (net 3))
 (segment (start 142.7988 85.6772) (end 144.0135 85.6772) (width 0.8) (layer "F.Cu") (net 3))
 (segment (start 156.71038 85.941399) (end 156.71038 84.89442) (width 0.4) (layer "F.Cu") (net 3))
 (segment (start 159.9692 82.4215) (end 158.6085 82.4215) (width 1) (layer "F.Cu") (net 3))
 (segment (start 149.41042 84.89442) (end 149.4028 84.8868) (width 0.4) (layer "F.Cu") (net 3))
 (segment (start 147.9296 85.3562) (end 147.1676 85.3562) (width 0.8) (layer "F.Cu") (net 3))
 (segment (start 149.4104 83.841401) (end 149.4104 84.8792) (width 0.4) (layer "F.Cu") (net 3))
 (segment (start 153.6192 80.3148) (end 152.9966 80.9374) (width 0.6) (layer "F.Cu") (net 3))
 (segment (start 144.8308 84.8599) (end 146.2415 84.8599) (width 0.8) (layer "F.Cu") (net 3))
 (segment (start 147.1676 85.3562) (end 146.4564 84.645) (width 0.8) (layer "F.Cu") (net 3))
 (segment (start 145.5659 77.7479) (end 145.9484 77.7479) (width 0.6) (layer "F.Cu") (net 3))
 (segment (start 140.5128 85.5472) (end 139.9032 84.9376) (width 0.8) (layer "F.Cu") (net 3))
 (segment (start 158.6085 82.4215) (end 158.2928 82.1058) (width 1) (layer "F.Cu") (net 3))
 (segment (start 149.4104 84.8792) (end 149.4028 84.8868) (width 0.4) (layer "F.Cu") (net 3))
 (segment (start 149.41042 85.941399) (end 149.41042 84.89442) (width 0.4) (layer "F.Cu") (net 3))
 (segment (start 156.7104 84.8792) (end 156.718 84.8868) (width 0.4) (layer "F.Cu") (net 3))
 (segment (start 144.7292 76.9112) (end 145.5659 77.7479) (width 0.6) (layer "F.Cu") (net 3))
 (segment (start 146.4564 85.4456) (end 146.4564 84.645) (width 0.8) (layer "F.Cu") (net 3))
 (segment (start 144.0135 85.6772) (end 144.8308 84.8599) (width 0.8) (layer "F.Cu") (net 3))
 (segment (start 146.2415 84.8599) (end 146.4564 84.645) (width 0.8) (layer "F.Cu") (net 3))
 (segment (start 143.51 76.9112) (end 144.7292 76.9112) (width 0.6) (layer "F.Cu") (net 3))
 (segment (start 143.1666 81.1906) (end 142.5448 81.1906) (width 0.6) (layer "F.Cu") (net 3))
 (segment (start 145.9484 78.486) (end 145.9484 77.7479) (width 0.6) (layer "F.Cu") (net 3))
 (segment (start 156.71038 84.89442) (end 156.718 84.8868) (width 0.4) (layer "F.Cu") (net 3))
 (segment (start 156.7104 83.841401) (end 156.7104 84.8792) (width 0.4) (layer "F.Cu") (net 3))
 (segment (start 143.2052 81.2292) (end 143.1666 81.1906) (width 0.6) (layer "F.Cu") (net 3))
 (segment (start 154.3105 80.3148) (end 153.6192 80.3148) (width 0.6) (layer "F.Cu") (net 3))
 (segment (start 142.4656 85.598) (end 142.4148 85.5472) (width 0.8) (layer "F.Cu") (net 3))
 (segment (start 142.4148 85.5472) (end 140.5128 85.5472) (width 0.8) (layer "F.Cu") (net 3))
 (via (at 139.32 85.52) (size 0.8) (drill 0.4) (layers "F.Cu" "B.Cu") (free yes) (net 3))
 (via (at 156.718 84.8868) (size 0.8) (drill 0.4) (layers "F.Cu" "B.Cu") (free yes) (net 3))
 (via (at 149.4028 84.8868) (size 0.8) (drill 0.4) (layers "F.Cu" "B.Cu") (free yes) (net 3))
 (via (at 140.49 85.52) (size 0.8) (drill 0.4) (layers "F.Cu" "B.Cu") (free yes) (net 3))
 (via (at 158.84 85.59) (size 0.8) (drill 0.4) (layers "F.Cu" "B.Cu") (free yes) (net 3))
 (via (at 156.62 77.25) (size 0.8) (drill 0.4) (layers "F.Cu" "B.Cu") (free yes) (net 3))
 (via (at 158.84 84.41) (size 0.8) (drill 0.4) (layers "F.Cu" "B.Cu") (free yes) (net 3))
 (via (at 143.2052 81.2292) (size 0.8) (drill 0.4) (layers "F.Cu" "B.Cu") (free yes) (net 3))
 (via (at 155.44 77.25) (size 0.8) (drill 0.4) (layers "F.Cu" "B.Cu") (free yes) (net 3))
 (via (at 156.62 76.07) (size 0.8) (drill 0.4) (layers "F.Cu" "B.Cu") (free yes) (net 3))
 (via (at 146.4564 85.4456) (size 0.8) (drill 0.4) (layers "F.Cu" "B.Cu") (free yes) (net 3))
 (via (at 160.02 84.41) (size 0.8) (drill 0.4) (layers "F.Cu" "B.Cu") (free yes) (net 3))
 (via (at 145.9484 78.486) (size 0.8) (drill 0.4) (layers "F.Cu" "B.Cu") (free yes) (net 3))
 (via (at 152.5524 81.5848) (size 0.8) (drill 0.4) (layers "F.Cu" "B.Cu") (free yes) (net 3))
 (via (at 140.49 84.35) (size 0.8) (drill 0.4) (layers "F.Cu" "B.Cu") (free yes) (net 3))
 (via (at 160.02 85.59) (size 0.8) (drill 0.4) (layers "F.Cu" "B.Cu") (free yes) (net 3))
 (via (at 139.31 84.35) (size 0.8) (drill 0.4) (layers "F.Cu" "B.Cu") (free yes) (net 3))
 (via (at 155.44 76.07) (size 0.8) (drill 0.4) (layers "F.Cu" "B.Cu") (free yes) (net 3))
 (segment (start 149.098 76.0785) (end 149.1865 75.99) (width 1) (layer "F.Cu") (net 1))
 (segment (start 149.098 76.0785) (end 148.9924 75.9729) (width 1) (layer "F.Cu") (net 1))
 (segment (start 148.9924 75.9729) (end 145.9564 75.9729) (width 1) (layer "F.Cu") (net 1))
 (segment (start 143.51 75.9612) (end 143.5217 75.9729) (width 0.8) (layer "F.Cu") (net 1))
 (segment (start 143.5217 75.9729) (end 145.9484 75.9729) (width 0.8) (layer "F.Cu") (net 1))
 (segment (start 151.936 75.99) (end 152.6032 76.6572) (width 1) (layer "F.Cu") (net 1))
 (segment (start 149.1865 75.99) (end 151.936 75.99) (width 1) (layer "F.Cu") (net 1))
 (segment (start 152.5524 79.3874) (end 151.6002 79.3874) (width 0.8) (layer "F.Cu") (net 9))
 (segment (start 155.448 83.0038) (end 155.448 79.797901) (width 0.4) (layer "F.Cu") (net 9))
 (segment (start 154.3105 79.3648) (end 152.575 79.3648) (width 0.8) (layer "F.Cu") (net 9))
 (segment (start 150.9512 80.0852) (end 150.9512 80.7212) (width 1) (layer "F.Cu") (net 9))
 (segment (start 155.014899 79.3648) (end 154.3105 79.3648) (width 0.4) (layer "F.Cu") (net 9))
 (segment (start 150.048 78.3535) (end 150.048 79.182) (width 1) (layer "F.Cu") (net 9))
 (segment (start 155.448 79.797901) (end 155.014899 79.3648) (width 0.4) (layer "F.Cu") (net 9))
 (segment (start 151.6002 79.3874) (end 150.9512 80.0364) (width 0.8) (layer "F.Cu") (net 9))
 (segment (start 150.9512 80.0364) (end 150.9512 80.7212) (width 0.8) (layer "F.Cu") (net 9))
 (segment (start 150.048 79.182) (end 150.9512 80.0852) (width 1) (layer "F.Cu") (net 9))
 (segment (start 159.9184 80.5957) (end 159.9184 78.3584) (width 1) (layer "F.Cu") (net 5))
 (segment (start 159.9692 80.6465) (end 159.9184 80.5957) (width 1) (layer "F.Cu") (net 5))
 (segment (start 156.5855 79.3648) (end 156.8856 79.3648) (width 1) (layer "F.Cu") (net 5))
 (segment (start 159.9184 78.3584) (end 159.43 77.87) (width 1) (layer "F.Cu") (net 5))
 (segment (start 156.8856 79.3648) (end 158.0766 80.5558) (width 1) (layer "F.Cu") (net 5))
 (segment (start 158.2928 80.5558) (end 159.8785 80.5558) (width 1) (layer "F.Cu") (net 5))
 (segment (start 159.8785 80.5558) (end 159.9692 80.6465) (width 1) (layer "F.Cu") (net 5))
 (segment (start 158.0766 80.5558) (end 158.2928 80.5558) (width 1) (layer "F.Cu") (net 5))
 (segment (start 144.0028 77.8612) (end 143.51 77.8612) (width 0.6) (layer "F.Cu") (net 6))
 (segment (start 144.3989 79.6544) (end 144.3989 78.2573) (width 0.6) (layer "F.Cu") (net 6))
 (segment (start 144.3989 78.2573) (end 144.0028 77.8612) (width 0.6) (layer "F.Cu") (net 6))
 (segment (start 146.0114 81.28) (end 146.0114 79.6919) (width 0.6) (layer "F.Cu") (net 4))
 (segment (start 141.5796 78.5754) (end 142.5448 79.5406) (width 0.6) (layer "F.Cu") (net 7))
 (segment (start 141.5644 77.8612) (end 141.5796 77.8764) (width 0.6) (layer "F.Cu") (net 7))
 (segment (start 141.5796 77.8764) (end 141.5796 78.5754) (width 0.6) (layer "F.Cu") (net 7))
 (segment (start 140.396 75.9612) (end 139.446 76.9112) (width 1) (layer "F.Cu") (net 2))
 (segment (start 148.148 79.182) (end 147.6512 79.6788) (width 1) (layer "F.Cu") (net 2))
 (segment (start 146.3665 83.0849) (end 146.4564 82.995) (width 1) (layer "F.Cu") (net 2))
 (segment (start 139.446 76.9112) (end 139.446 80.264) (width 1) (layer "F.Cu") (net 2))
 (segment (start 141.235 75.9612) (end 140.396 75.9612) (width 1) (layer "F.Cu") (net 2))
 (segment (start 148.148 78.3535) (end 148.148 79.182) (width 1) (layer "F.Cu") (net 2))
 (segment (start 139.9032 81.1276) (end 141.6528 82.8772) (width 1) (layer "F.Cu") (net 2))
 (segment (start 146.4564 82.9056) (end 146.4564 82.995) (width 1) (layer "F.Cu") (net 2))
 (segment (start 142.7988 82.8772) (end 142.9796 83.058) (width 1) (layer "F.Cu") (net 2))
 (segment (start 141.6528 82.8772) (end 142.7988 82.8772) (width 1) (layer "F.Cu") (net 2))
 (segment (start 144.8039 83.058) (end 144.8308 83.0849) (width 1) (layer "F.Cu") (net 2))
 (segment (start 144.3736 81.2922) (end 144.3736 83.0072) (width 0.6) (layer "F.Cu") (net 2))
 (segment (start 144.8308 83.0849) (end 146.3665 83.0849) (width 1) (layer "F.Cu") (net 2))
 (segment (start 147.6512 79.6788) (end 147.6512 80.7212) (width 1) (layer "F.Cu") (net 2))
 (segment (start 147.6512 81.7108) (end 146.4564 82.9056) (width 1) (layer "F.Cu") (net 2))
 (segment (start 139.446 80.264) (end 139.8524 80.6704) (width 1) (layer "F.Cu") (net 2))
 (segment (start 142.9796 83.058) (end 144.8039 83.058) (width 1) (layer "F.Cu") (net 2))
 (segment (start 147.6512 80.7212) (end 147.6512 81.7108) (width 1) (layer "F.Cu") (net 2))
 (segment (start 153.8104 83.1414) (end 153.8104 81.546) (width 0.4) (layer "F.Cu") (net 8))
 (segment (start 153.8104 81.546) (end 153.99 81.3664) (width 0.4) (layer "F.Cu") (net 8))
 (segment (start 147.9296 83.4644) (end 147.9296 83.7062) (width 0.4) (layer "F.Cu") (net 8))
 (segment (start 148.7932 82.6008) (end 147.9296 83.4644) (width 0.4) (layer "F.Cu") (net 8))
 (segment (start 150.810397 82.6008) (end 148.7932 82.6008) (width 0.4) (layer "F.Cu") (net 8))
 (segment (start 153.8104 83.1414) (end 150.810397 83.1414) (width 0.4) (layer "F.Cu") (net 8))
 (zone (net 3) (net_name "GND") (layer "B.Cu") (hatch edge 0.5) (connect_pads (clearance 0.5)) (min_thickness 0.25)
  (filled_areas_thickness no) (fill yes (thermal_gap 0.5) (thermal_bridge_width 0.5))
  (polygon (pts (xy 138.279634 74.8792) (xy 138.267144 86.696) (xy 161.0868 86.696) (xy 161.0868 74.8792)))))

